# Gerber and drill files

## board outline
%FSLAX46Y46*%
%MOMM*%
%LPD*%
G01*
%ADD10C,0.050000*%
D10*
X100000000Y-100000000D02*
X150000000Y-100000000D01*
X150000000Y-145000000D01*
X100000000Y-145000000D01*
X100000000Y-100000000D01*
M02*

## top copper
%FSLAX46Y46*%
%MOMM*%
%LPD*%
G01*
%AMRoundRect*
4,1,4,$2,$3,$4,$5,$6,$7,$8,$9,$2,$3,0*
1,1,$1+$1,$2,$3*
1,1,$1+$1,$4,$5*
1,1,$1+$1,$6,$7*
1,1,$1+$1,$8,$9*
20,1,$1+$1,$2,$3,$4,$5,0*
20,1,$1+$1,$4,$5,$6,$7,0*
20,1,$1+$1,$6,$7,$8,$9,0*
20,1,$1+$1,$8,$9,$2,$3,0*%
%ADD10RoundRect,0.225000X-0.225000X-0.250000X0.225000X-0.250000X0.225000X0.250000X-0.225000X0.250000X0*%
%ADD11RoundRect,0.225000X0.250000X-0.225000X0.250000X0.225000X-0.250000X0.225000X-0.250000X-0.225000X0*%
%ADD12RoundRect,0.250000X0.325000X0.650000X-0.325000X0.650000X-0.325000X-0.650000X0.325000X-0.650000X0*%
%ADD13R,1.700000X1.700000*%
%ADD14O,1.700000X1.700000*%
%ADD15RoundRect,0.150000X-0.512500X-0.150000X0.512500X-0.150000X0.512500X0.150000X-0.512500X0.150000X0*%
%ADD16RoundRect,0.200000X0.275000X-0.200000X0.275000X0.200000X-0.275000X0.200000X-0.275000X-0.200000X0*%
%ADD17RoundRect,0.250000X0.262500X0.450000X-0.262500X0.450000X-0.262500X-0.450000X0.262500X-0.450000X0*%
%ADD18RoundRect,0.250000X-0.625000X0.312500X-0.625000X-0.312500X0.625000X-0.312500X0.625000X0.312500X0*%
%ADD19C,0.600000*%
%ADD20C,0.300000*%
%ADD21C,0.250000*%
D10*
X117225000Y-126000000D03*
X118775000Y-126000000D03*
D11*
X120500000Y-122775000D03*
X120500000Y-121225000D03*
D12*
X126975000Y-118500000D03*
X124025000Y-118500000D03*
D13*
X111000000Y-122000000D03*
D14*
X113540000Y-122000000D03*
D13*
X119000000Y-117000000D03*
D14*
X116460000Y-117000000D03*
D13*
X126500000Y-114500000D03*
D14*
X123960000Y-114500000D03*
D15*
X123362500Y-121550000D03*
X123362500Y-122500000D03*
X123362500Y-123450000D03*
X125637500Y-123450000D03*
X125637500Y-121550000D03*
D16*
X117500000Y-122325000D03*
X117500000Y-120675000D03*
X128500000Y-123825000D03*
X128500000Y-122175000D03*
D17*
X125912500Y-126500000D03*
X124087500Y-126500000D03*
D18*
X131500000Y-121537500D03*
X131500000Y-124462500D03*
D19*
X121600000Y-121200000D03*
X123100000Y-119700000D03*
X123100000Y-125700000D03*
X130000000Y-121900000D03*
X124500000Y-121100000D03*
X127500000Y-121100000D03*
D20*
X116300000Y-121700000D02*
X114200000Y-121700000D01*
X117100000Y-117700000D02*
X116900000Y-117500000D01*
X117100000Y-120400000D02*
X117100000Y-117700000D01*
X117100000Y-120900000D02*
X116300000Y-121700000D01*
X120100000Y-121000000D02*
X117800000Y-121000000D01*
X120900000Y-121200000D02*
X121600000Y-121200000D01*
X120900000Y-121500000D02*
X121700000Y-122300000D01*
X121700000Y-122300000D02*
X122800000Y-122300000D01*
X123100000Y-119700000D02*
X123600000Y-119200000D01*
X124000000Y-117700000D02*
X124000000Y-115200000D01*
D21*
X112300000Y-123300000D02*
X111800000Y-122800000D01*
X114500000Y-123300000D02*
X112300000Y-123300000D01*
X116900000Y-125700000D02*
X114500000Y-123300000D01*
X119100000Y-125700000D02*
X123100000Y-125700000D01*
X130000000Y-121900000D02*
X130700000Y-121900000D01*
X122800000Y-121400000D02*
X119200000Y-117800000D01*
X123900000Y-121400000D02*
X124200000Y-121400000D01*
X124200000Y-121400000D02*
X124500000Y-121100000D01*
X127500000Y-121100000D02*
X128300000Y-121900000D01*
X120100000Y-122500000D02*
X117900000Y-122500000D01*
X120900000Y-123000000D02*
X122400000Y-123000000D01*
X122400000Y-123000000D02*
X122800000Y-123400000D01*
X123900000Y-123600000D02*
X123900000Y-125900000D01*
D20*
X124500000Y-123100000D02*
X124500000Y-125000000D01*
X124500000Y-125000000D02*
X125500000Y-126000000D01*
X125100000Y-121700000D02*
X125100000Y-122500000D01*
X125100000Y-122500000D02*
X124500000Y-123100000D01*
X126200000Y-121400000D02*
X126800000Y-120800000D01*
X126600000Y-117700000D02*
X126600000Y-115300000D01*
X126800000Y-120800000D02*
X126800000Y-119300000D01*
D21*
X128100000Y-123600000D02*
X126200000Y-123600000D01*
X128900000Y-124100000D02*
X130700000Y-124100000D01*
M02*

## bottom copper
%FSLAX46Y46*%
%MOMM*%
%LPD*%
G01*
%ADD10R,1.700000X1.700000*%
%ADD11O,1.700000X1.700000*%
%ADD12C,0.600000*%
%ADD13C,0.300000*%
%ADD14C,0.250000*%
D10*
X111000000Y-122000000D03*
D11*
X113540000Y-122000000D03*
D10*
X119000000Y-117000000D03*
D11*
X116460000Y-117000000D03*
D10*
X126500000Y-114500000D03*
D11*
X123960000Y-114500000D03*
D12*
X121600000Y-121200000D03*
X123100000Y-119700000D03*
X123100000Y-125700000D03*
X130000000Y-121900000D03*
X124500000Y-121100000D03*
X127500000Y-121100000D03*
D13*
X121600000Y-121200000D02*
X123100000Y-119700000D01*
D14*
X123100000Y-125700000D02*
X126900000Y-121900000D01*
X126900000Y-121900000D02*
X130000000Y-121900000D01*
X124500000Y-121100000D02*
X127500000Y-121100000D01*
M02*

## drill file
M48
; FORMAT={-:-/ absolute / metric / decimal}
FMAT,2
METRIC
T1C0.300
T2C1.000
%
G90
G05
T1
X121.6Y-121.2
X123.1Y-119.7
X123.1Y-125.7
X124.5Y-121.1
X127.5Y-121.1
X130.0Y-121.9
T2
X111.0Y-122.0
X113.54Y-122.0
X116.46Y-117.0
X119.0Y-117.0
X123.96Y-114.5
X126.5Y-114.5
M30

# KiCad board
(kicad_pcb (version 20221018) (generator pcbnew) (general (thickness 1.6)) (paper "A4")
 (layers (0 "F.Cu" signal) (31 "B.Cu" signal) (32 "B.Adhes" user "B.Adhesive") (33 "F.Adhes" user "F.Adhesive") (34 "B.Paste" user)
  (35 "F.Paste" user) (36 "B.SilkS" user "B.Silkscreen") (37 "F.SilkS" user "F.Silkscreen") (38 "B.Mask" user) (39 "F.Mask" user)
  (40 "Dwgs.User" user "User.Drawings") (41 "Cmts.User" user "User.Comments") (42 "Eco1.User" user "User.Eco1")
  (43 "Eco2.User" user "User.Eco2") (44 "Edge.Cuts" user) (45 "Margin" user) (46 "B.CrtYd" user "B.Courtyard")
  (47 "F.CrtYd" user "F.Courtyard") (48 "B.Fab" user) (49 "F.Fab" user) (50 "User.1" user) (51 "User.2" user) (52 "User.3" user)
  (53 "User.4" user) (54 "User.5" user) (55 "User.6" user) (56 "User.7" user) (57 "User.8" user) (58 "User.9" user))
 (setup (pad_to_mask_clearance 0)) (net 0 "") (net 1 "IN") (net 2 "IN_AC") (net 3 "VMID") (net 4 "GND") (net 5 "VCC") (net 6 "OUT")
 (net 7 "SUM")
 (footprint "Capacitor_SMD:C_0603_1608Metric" (layer "F.Cu") (at 118 126)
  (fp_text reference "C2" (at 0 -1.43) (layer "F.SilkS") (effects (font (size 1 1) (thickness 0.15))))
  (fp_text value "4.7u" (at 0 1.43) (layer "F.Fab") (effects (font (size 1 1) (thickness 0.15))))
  (pad "1" smd roundrect (at -0.775 0) (size 0.9 0.95) (layers "F.Cu" "F.Paste" "F.Mask") (roundrect_rratio 0.25) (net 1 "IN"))
  (pad "2" smd roundrect (at 0.775 0) (size 0.9 0.95) (layers "F.Cu" "F.Paste" "F.Mask") (roundrect_rratio 0.25) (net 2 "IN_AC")))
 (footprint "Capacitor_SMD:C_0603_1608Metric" (layer "F.Cu") (at 120.5 122 90)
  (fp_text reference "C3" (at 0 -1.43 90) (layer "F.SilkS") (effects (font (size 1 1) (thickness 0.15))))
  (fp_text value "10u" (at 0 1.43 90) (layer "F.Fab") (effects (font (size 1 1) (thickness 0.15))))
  (pad "1" smd roundrect (at -0.775 0 90) (size 0.9 0.95) (layers "F.Cu" "F.Paste" "F.Mask") (roundrect_rratio 0.25) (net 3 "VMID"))
  (pad "2" smd roundrect (at 0.775 0 90) (size 0.9 0.95) (layers "F.Cu" "F.Paste" "F.Mask") (roundrect_rratio 0.25) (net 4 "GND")))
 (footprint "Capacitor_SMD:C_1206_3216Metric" (layer "F.Cu") (at 125.5 118.5 180)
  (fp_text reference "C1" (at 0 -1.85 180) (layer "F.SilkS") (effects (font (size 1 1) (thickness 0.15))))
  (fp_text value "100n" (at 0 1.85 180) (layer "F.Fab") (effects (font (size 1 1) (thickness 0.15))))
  (pad "1" smd roundrect (at -1.475 0 180) (size 1.15 1.8) (layers "F.Cu" "F.Paste" "F.Mask") (roundrect_rratio 0.217391) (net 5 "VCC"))
  (pad "2" smd roundrect (at 1.475 0 180) (size 1.15 1.8) (layers "F.Cu" "F.Paste" "F.Mask") (roundrect_rratio 0.217391) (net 4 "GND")))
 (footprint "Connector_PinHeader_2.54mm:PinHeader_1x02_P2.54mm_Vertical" (layer "F.Cu") (at 111 122 90)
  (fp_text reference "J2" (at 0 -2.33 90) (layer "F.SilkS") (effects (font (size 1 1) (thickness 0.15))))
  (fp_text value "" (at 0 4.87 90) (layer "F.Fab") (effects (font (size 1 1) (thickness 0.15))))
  (pad "1" thru_hole rect (at 0 0 90) (size 1.7 1.7) (drill 1) (layers "*.Cu" "*.Mask") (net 1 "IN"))
  (pad "2" thru_hole oval (at 0 2.54 90) (size 1.7 1.7) (drill 1) (layers "*.Cu" "*.Mask") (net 4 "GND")))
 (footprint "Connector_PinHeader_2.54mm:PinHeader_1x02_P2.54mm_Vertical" (layer "F.Cu") (at 119 117 -90)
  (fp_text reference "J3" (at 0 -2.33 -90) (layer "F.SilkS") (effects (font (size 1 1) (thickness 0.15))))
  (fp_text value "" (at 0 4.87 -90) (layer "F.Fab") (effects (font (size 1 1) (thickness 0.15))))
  (pad "1" thru_hole rect (at 0 0 270) (size 1.7 1.7) (drill 1) (layers "*.Cu" "*.Mask") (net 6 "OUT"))
  (pad "2" thru_hole oval (at 0 2.54 270) (size 1.7 1.7) (drill 1) (layers "*.Cu" "*.Mask") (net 4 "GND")))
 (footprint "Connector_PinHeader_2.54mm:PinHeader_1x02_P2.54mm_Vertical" (layer "F.Cu") (at 126.5 114.5 -90)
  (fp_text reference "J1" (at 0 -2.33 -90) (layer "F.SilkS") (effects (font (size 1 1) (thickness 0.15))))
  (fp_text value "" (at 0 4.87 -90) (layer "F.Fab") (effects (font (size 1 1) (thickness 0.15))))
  (pad "1" thru_hole rect (at 0 0 270) (size 1.7 1.7) (drill 1) (layers "*.Cu" "*.Mask") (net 5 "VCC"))
  (pad "2" thru_hole oval (at 0 2.54 270) (size 1.7 1.7) (drill 1) (layers "*.Cu" "*.Mask") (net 4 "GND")))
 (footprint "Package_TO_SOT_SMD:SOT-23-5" (layer "F.Cu") (at 124.5 122.5)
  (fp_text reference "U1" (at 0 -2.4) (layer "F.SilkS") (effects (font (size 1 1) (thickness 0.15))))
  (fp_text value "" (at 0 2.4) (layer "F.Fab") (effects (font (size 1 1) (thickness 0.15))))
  (pad "1" smd roundrect (at -1.1375 -0.95) (size 1.325 0.6) (layers "F.Cu" "F.Paste" "F.Mask") (roundrect_rratio 0.25) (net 6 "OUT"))
  (pad "2" smd roundrect (at -1.1375 0) (size 1.325 0.6) (layers "F.Cu" "F.Paste" "F.Mask") (roundrect_rratio 0.25) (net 4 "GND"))
  (pad "3" smd roundrect (at -1.1375 0.95) (size 1.325 0.6) (layers "F.Cu" "F.Paste" "F.Mask") (roundrect_rratio 0.25) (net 3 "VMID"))
  (pad "4" smd roundrect (at 1.1375 0.95) (size 1.325 0.6) (layers "F.Cu" "F.Paste" "F.Mask") (roundrect_rratio 0.25) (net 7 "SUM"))
  (pad "5" smd roundrect (at 1.1375 -0.95) (size 1.325 0.6) (layers "F.Cu" "F.Paste" "F.Mask") (roundrect_rratio 0.25) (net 5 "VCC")))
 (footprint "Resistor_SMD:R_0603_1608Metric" (layer "F.Cu") (at 117.5 121.5 90)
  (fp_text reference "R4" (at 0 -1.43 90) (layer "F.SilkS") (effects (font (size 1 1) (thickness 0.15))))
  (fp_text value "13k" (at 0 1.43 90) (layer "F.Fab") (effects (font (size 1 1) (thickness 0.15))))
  (pad "1" smd roundrect (at -0.825 0 90) (size 0.8 0.95) (layers "F.Cu" "F.Paste" "F.Mask") (roundrect_rratio 0.25) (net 3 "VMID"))
  (pad "2" smd roundrect (at 0.825 0 90) (size 0.8 0.95) (layers "F.Cu" "F.Paste" "F.Mask") (roundrect_rratio 0.25) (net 4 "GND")))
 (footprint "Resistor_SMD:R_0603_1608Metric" (layer "F.Cu") (at 128.5 123 90)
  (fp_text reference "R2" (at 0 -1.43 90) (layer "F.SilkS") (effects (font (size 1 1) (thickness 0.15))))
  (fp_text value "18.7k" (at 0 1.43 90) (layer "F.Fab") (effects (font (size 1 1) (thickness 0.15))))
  (pad "1" smd roundrect (at -0.825 0 90) (size 0.8 0.95) (layers "F.Cu" "F.Paste" "F.Mask") (roundrect_rratio 0.25) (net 7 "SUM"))
  (pad "2" smd roundrect (at 0.825 0 90) (size 0.8 0.95) (layers "F.Cu" "F.Paste" "F.Mask") (roundrect_rratio 0.25) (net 6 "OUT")))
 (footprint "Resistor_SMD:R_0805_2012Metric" (layer "F.Cu") (at 125 126.5 180)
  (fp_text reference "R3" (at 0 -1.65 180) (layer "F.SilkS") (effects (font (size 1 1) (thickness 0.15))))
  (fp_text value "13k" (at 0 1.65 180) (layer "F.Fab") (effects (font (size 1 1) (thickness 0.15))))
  (pad "1" smd roundrect (at -0.9125 0 180) (size 1.025 1.4) (layers "F.Cu" "F.Paste" "F.Mask") (roundrect_rratio 0.243902) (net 5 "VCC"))
  (pad "2" smd roundrect (at 0.9125 0 180) (size 1.025 1.4) (layers "F.Cu" "F.Paste" "F.Mask") (roundrect_rratio 0.243902) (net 3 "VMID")))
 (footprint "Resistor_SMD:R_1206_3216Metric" (layer "F.Cu") (at 131.5 123 -90)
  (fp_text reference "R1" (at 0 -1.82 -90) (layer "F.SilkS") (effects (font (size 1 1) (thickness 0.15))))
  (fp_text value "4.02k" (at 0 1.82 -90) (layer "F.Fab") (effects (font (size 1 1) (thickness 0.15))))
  (pad "1" smd roundrect (at -1.4625 0 270) (size 1.125 1.75) (layers "F.Cu" "F.Paste" "F.Mask") (roundrect_rratio 0.222222) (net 2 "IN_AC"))
  (pad "2" smd roundrect (at 1.4625 0 270) (size 1.125 1.75) (layers "F.Cu" "F.Paste" "F.Mask") (roundrect_rratio 0.222222) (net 7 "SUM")))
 (gr_rect (start 100 100) (end 150 145) (stroke (width 0.05) (type default)) (fill none) (layer "Edge.Cuts"))
 (segment (start 116.3 121.7) (end 114.2 121.7) (width 0.3) (layer "F.Cu") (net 4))
 (segment (start 117.1 117.7) (end 116.9 117.5) (width 0.3) (layer "F.Cu") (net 4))
 (segment (start 117.1 120.4) (end 117.1 117.7) (width 0.3) (layer "F.Cu") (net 4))
 (segment (start 117.1 120.9) (end 116.3 121.7) (width 0.3) (layer "F.Cu") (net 4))
 (segment (start 120.1 121) (end 117.8 121) (width 0.3) (layer "F.Cu") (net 4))
 (segment (start 120.9 121.2) (end 121.6 121.2) (width 0.3) (layer "F.Cu") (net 4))
 (segment (start 120.9 121.5) (end 121.7 122.3) (width 0.3) (layer "F.Cu") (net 4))
 (segment (start 121.7 122.3) (end 122.8 122.3) (width 0.3) (layer "F.Cu") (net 4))
 (segment (start 123.1 119.7) (end 123.6 119.2) (width 0.3) (layer "F.Cu") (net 4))
 (segment (start 124 117.7) (end 124 115.2) (width 0.3) (layer "F.Cu") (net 4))
 (via (at 121.6 121.2) (size 0.6) (drill 0.3) (layers "F.Cu" "B.Cu") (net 4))
 (via (at 123.1 119.7) (size 0.6) (drill 0.3) (layers "F.Cu" "B.Cu") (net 4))
 (segment (start 112.3 123.3) (end 111.8 122.8) (width 0.25) (layer "F.Cu") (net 1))
 (segment (start 114.5 123.3) (end 112.3 123.3) (width 0.25) (layer "F.Cu") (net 1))
 (segment (start 116.9 125.7) (end 114.5 123.3) (width 0.25) (layer "F.Cu") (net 1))
 (segment (start 119.1 125.7) (end 123.1 125.7) (width 0.25) (layer "F.Cu") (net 2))
 (segment (start 121.6 121.2) (end 123.1 119.7) (width 0.3) (layer "B.Cu") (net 4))
 (segment (start 130 121.9) (end 130.7 121.9) (width 0.25) (layer "F.Cu") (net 2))
 (via (at 123.1 125.7) (size 0.6) (drill 0.3) (layers "F.Cu" "B.Cu") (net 2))
 (via (at 130 121.9) (size 0.6) (drill 0.3) (layers "F.Cu" "B.Cu") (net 2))
 (segment (start 122.8 121.4) (end 119.2 117.8) (width 0.25) (layer "F.Cu") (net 6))
 (segment (start 123.1 125.7) (end 126.9 121.9) (width 0.25) (layer "B.Cu") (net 2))
 (segment (start 123.9 121.4) (end 124.2 121.4) (width 0.25) (layer "F.Cu") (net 6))
 (segment (start 124.2 121.4) (end 124.5 121.1) (width 0.25) (layer "F.Cu") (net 6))
 (segment (start 126.9 121.9) (end 130 121.9) (width 0.25) (layer "B.Cu") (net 2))
 (segment (start 127.5 121.1) (end 128.3 121.9) (width 0.25) (layer "F.Cu") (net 6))
 (via (at 124.5 121.1) (size 0.6) (drill 0.3) (layers "F.Cu" "B.Cu") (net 6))
 (via (at 127.5 121.1) (size 0.6) (drill 0.3) (layers "F.Cu" "B.Cu") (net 6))
 (segment (start 120.1 122.5) (end 117.9 122.5) (width 0.25) (layer "F.Cu") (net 3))
 (segment (start 120.9 123) (end 122.4 123) (width 0.25) (layer "F.Cu") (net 3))
 (segment (start 122.4 123) (end 122.8 123.4) (width 0.25) (layer "F.Cu") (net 3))
 (segment (start 123.9 123.6) (end 123.9 125.9) (width 0.25) (layer "F.Cu") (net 3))
 (segment (start 124.5 121.1) (end 127.5 121.1) (width 0.25) (layer "B.Cu") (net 6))
 (segment (start 124.5 123.1) (end 124.5 125) (width 0.3) (layer "F.Cu") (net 5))
 (segment (start 124.5 125) (end 125.5 126) (width 0.3) (layer "F.Cu") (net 5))
 (segment (start 125.1 121.7) (end 125.1 122.5) (width 0.3) (layer "F.Cu") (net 5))
 (segment (start 125.1 122.5) (end 124.5 123.1) (width 0.3) (layer "F.Cu") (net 5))
 (segment (start 126.2 121.4) (end 126.8 120.8) (width 0.3) (layer "F.Cu") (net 5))
 (segment (start 126.6 117.7) (end 126.6 115.3) (width 0.3) (layer "F.Cu") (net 5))
 (segment (start 126.8 120.8) (end 126.8 119.3) (width 0.3) (layer "F.Cu") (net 5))
 (segment (start 128.1 123.6) (end 126.2 123.6) (width 0.25) (layer "F.Cu") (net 7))
 (segment (start 128.9 124.1) (end 130.7 124.1) (width 0.25) (layer "F.Cu") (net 7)))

